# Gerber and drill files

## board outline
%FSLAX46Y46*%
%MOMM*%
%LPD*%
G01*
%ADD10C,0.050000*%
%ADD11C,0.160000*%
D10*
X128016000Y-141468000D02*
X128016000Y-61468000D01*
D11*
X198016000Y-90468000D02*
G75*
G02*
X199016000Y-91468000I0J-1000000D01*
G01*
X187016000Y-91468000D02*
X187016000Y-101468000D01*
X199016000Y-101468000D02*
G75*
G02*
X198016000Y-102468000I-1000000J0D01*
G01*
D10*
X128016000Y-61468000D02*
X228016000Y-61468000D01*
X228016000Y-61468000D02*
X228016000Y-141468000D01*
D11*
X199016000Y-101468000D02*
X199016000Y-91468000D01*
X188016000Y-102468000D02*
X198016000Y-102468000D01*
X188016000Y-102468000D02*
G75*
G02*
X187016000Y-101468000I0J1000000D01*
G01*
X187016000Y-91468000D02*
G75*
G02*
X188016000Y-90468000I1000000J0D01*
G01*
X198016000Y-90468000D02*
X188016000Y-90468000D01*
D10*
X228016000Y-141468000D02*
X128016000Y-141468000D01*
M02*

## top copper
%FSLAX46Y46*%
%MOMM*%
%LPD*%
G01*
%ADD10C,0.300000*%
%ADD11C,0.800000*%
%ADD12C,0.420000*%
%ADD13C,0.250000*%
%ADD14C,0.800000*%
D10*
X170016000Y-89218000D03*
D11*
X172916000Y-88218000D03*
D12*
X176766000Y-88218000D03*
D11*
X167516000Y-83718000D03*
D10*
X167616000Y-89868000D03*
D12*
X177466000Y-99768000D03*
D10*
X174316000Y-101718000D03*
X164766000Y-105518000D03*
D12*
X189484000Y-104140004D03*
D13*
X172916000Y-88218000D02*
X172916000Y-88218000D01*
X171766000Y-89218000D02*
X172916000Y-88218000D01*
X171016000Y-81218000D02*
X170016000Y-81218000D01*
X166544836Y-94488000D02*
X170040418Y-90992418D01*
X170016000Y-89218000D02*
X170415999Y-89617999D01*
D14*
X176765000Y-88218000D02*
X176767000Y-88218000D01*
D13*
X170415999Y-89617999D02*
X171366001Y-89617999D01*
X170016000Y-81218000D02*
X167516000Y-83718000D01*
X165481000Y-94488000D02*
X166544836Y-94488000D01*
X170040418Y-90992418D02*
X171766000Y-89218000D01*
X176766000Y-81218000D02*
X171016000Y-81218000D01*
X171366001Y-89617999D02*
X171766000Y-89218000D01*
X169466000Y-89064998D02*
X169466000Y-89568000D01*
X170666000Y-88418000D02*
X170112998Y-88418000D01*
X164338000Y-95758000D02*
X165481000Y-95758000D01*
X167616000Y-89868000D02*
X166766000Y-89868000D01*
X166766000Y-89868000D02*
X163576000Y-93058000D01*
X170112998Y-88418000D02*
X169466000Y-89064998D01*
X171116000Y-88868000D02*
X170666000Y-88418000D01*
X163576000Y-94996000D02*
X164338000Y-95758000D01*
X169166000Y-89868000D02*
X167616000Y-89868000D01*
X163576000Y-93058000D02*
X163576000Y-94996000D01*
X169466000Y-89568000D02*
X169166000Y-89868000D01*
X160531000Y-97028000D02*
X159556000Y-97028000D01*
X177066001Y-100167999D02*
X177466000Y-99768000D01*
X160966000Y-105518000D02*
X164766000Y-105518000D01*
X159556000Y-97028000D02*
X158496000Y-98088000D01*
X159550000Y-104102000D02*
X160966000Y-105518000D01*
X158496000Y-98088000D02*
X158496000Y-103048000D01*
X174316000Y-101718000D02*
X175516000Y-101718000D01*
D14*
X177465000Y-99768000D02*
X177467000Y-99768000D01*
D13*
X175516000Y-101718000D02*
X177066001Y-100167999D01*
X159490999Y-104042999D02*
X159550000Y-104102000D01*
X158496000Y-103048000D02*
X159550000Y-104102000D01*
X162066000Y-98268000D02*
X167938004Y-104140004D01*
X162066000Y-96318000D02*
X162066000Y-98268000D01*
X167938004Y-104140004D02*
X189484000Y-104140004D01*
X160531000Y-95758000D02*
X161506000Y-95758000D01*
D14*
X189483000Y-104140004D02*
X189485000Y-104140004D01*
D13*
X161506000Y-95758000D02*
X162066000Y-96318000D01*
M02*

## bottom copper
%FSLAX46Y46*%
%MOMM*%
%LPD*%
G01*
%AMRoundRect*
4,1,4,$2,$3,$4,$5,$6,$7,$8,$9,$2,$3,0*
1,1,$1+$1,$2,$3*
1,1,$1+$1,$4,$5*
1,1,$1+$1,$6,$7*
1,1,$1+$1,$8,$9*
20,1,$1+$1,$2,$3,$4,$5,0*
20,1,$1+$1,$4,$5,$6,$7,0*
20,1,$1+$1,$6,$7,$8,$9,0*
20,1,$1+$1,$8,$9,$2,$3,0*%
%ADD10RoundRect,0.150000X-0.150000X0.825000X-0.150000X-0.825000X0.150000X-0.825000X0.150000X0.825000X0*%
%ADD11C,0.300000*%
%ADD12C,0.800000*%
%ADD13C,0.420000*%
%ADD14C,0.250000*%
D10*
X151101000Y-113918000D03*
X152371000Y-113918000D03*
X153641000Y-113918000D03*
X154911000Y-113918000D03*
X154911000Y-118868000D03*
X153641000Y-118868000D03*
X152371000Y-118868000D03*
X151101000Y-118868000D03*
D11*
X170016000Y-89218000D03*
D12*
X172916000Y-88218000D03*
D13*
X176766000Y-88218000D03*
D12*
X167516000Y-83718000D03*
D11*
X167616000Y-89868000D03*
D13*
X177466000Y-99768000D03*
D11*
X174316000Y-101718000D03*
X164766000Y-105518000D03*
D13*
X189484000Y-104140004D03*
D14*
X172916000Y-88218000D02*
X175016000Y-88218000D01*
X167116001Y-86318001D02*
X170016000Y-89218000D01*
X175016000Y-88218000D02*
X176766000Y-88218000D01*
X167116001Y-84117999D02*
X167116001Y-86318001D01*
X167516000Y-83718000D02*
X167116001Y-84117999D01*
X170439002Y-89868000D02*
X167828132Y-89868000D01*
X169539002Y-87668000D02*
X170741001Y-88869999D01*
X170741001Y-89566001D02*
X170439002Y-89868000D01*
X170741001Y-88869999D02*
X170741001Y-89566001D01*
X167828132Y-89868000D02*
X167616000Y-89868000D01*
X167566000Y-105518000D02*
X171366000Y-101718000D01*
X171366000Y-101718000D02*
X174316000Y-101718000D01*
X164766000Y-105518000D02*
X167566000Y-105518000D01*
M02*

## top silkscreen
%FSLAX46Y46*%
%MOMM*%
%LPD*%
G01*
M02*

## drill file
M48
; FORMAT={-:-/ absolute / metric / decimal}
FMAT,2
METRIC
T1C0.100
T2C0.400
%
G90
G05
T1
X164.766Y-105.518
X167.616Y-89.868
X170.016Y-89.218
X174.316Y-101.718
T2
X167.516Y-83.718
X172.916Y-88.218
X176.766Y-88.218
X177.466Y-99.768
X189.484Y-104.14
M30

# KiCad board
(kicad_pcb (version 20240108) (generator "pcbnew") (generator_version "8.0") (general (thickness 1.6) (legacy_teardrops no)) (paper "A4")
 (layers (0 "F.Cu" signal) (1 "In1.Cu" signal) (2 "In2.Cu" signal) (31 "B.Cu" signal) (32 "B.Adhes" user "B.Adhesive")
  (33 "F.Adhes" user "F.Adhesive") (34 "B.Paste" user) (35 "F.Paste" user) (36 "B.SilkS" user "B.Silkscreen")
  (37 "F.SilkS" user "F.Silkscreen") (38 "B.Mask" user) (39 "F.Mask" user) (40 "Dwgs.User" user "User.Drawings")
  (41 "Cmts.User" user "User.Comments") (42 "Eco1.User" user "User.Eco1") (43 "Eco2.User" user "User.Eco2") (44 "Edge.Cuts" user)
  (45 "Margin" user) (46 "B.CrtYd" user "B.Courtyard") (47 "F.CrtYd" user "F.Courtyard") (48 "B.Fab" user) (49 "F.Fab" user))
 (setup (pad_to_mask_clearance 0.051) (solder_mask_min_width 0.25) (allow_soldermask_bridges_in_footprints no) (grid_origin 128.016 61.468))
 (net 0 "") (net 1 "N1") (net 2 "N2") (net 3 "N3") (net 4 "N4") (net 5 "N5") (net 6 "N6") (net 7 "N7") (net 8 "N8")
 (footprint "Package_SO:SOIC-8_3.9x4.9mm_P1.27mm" (layer "B.Cu") (at 153.006 116.393 -90)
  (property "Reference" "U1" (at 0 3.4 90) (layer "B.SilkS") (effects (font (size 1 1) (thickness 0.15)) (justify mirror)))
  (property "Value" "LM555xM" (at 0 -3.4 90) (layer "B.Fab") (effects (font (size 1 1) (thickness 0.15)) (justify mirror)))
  (pad "1" smd roundrect (at -2.475 1.905 270) (size 1.95 0.6) (layers "B.Cu" "B.Paste" "B.Mask") (roundrect_rratio 0.25) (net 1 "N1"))
  (pad "2" smd roundrect (at -2.475 0.635 270) (size 1.95 0.6) (layers "B.Cu" "B.Paste" "B.Mask") (roundrect_rratio 0.25) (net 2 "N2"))
  (pad "3" smd roundrect (at -2.475 -0.635 270) (size 1.95 0.6) (layers "B.Cu" "B.Paste" "B.Mask") (roundrect_rratio 0.25) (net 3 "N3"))
  (pad "4" smd roundrect (at -2.475 -1.905 270) (size 1.95 0.6) (layers "B.Cu" "B.Paste" "B.Mask") (roundrect_rratio 0.25) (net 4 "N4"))
  (pad "5" smd roundrect (at 2.475 -1.905 270) (size 1.95 0.6) (layers "B.Cu" "B.Paste" "B.Mask") (roundrect_rratio 0.25) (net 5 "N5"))
  (pad "6" smd roundrect (at 2.475 -0.635 270) (size 1.95 0.6) (layers "B.Cu" "B.Paste" "B.Mask") (roundrect_rratio 0.25) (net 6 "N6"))
  (pad "7" smd roundrect (at 2.475 0.635 270) (size 1.95 0.6) (layers "B.Cu" "B.Paste" "B.Mask") (roundrect_rratio 0.25) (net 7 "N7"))
  (pad "8" smd roundrect (at 2.475 1.905 270) (size 1.95 0.6) (layers "B.Cu" "B.Paste" "B.Mask") (roundrect_rratio 0.25) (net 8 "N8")))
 (gr_line (start 128.016 141.468) (end 128.016 61.468) (stroke (width 0.05) (type solid)) (layer "Edge.Cuts"))
 (gr_arc (start 198.016 90.468) (mid 198.723107 90.760893) (end 199.016 91.468) (stroke (width 0.16) (type solid)) (layer "Edge.Cuts"))
 (gr_line (start 187.016 91.468) (end 187.016 101.468) (stroke (width 0.16) (type solid)) (layer "Edge.Cuts"))
 (gr_arc (start 199.016 101.468) (mid 198.723107 102.175107) (end 198.016 102.468) (stroke (width 0.16) (type solid)) (layer "Edge.Cuts"))
 (gr_line (start 128.016 61.468) (end 228.016 61.468) (stroke (width 0.05) (type solid)) (layer "Edge.Cuts"))
 (gr_line (start 228.016 61.468) (end 228.016 141.468) (stroke (width 0.05) (type solid)) (layer "Edge.Cuts"))
 (gr_line (start 199.016 101.468) (end 199.016 91.468) (stroke (width 0.16) (type solid)) (layer "Edge.Cuts"))
 (gr_line (start 188.016 102.468) (end 198.016 102.468) (stroke (width 0.16) (type solid)) (layer "Edge.Cuts"))
 (gr_arc (start 188.016 102.468) (mid 187.308893 102.175107) (end 187.016 101.468) (stroke (width 0.16) (type solid)) (layer "Edge.Cuts"))
 (gr_arc (start 187.016 91.468) (mid 187.308893 90.760893) (end 188.016 90.468) (stroke (width 0.16) (type solid)) (layer "Edge.Cuts"))
 (gr_line (start 198.016 90.468) (end 188.016 90.468) (stroke (width 0.16) (type solid)) (layer "Edge.Cuts"))
 (gr_line (start 228.016 141.468) (end 128.016 141.468) (stroke (width 0.05) (type solid)) (layer "Edge.Cuts"))
 (segment (start 172.916 88.218) (end 172.916 88.218) (width 0.25) (layer "F.Cu") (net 8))
 (segment (start 171.766 89.218) (end 172.916 88.218) (width 0.25) (layer "F.Cu") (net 8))
 (segment (start 171.016 81.218) (end 170.016 81.218) (width 0.25) (layer "F.Cu") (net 8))
 (segment (start 166.544836 94.488) (end 170.040418 90.992418) (width 0.25) (layer "F.Cu") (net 8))
 (segment (start 170.016 89.218) (end 170.415999 89.617999) (width 0.25) (layer "F.Cu") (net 8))
 (segment (start 176.765 88.218) (end 176.767 88.218) (width 0.8) (layer "F.Cu") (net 8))
 (segment (start 170.415999 89.617999) (end 171.366001 89.617999) (width 0.25) (layer "F.Cu") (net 8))
 (segment (start 170.016 81.218) (end 167.516 83.718) (width 0.25) (layer "F.Cu") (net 8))
 (segment (start 165.481 94.488) (end 166.544836 94.488) (width 0.25) (layer "F.Cu") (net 8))
 (segment (start 170.040418 90.992418) (end 171.766 89.218) (width 0.25) (layer "F.Cu") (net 8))
 (segment (start 176.766 81.218) (end 171.016 81.218) (width 0.25) (layer "F.Cu") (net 8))
 (segment (start 171.366001 89.617999) (end 171.766 89.218) (width 0.25) (layer "F.Cu") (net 8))
 (via (at 170.016 89.218) (size 0.3) (drill 0.1) (layers "F.Cu" "B.Cu") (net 8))
 (via (at 172.916 88.218) (size 0.8) (drill 0.4) (layers "F.Cu" "B.Cu") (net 8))
 (via (at 176.766 88.218) (size 0.42) (drill 0.4) (layers "F.Cu" "B.Cu") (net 8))
 (via (at 167.516 83.718) (size 0.8) (drill 0.4) (layers "F.Cu" "B.Cu") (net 8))
 (segment (start 172.916 88.218) (end 175.016 88.218) (width 0.25) (layer "B.Cu") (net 8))
 (segment (start 167.116001 86.318001) (end 170.016 89.218) (width 0.25) (layer "B.Cu") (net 8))
 (segment (start 175.016 88.218) (end 176.766 88.218) (width 0.25) (layer "B.Cu") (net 8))
 (segment (start 167.116001 84.117999) (end 167.116001 86.318001) (width 0.25) (layer "B.Cu") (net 8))
 (segment (start 167.516 83.718) (end 167.116001 84.117999) (width 0.25) (layer "B.Cu") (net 8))
 (segment (start 169.466 89.064998) (end 169.466 89.568) (width 0.25) (layer "F.Cu") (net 7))
 (segment (start 170.666 88.418) (end 170.112998 88.418) (width 0.25) (layer "F.Cu") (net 7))
 (segment (start 164.338 95.758) (end 165.481 95.758) (width 0.25) (layer "F.Cu") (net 7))
 (segment (start 167.616 89.868) (end 166.766 89.868) (width 0.25) (layer "F.Cu") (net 7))
 (segment (start 166.766 89.868) (end 163.576 93.058) (width 0.25) (layer "F.Cu") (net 7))
 (segment (start 170.112998 88.418) (end 169.466 89.064998) (width 0.25) (layer "F.Cu") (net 7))
 (segment (start 171.116 88.868) (end 170.666 88.418) (width 0.25) (layer "F.Cu") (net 7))
 (segment (start 163.576 94.996) (end 164.338 95.758) (width 0.25) (layer "F.Cu") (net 7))
 (segment (start 169.166 89.868) (end 167.616 89.868) (width 0.25) (layer "F.Cu") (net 7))
 (segment (start 163.576 93.058) (end 163.576 94.996) (width 0.25) (layer "F.Cu") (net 7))
 (segment (start 169.466 89.568) (end 169.166 89.868) (width 0.25) (layer "F.Cu") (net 7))
 (via (at 167.616 89.868) (size 0.3) (drill 0.1) (layers "F.Cu" "B.Cu") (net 7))
 (segment (start 170.439002 89.868) (end 167.828132 89.868) (width 0.25) (layer "B.Cu") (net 7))
 (segment (start 169.539002 87.668) (end 170.741001 88.869999) (width 0.25) (layer "B.Cu") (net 7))
 (segment (start 170.741001 89.566001) (end 170.439002 89.868) (width 0.25) (layer "B.Cu") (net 7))
 (segment (start 170.741001 88.869999) (end 170.741001 89.566001) (width 0.25) (layer "B.Cu") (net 7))
 (segment (start 167.828132 89.868) (end 167.616 89.868) (width 0.25) (layer "B.Cu") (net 7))
 (segment (start 160.531 97.028) (end 159.556 97.028) (width 0.25) (layer "F.Cu") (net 3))
 (segment (start 177.066001 100.167999) (end 177.466 99.768) (width 0.25) (layer "F.Cu") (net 3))
 (segment (start 160.966 105.518) (end 164.766 105.518) (width 0.25) (layer "F.Cu") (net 3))
 (segment (start 159.556 97.028) (end 158.496 98.088) (width 0.25) (layer "F.Cu") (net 3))
 (segment (start 159.55 104.102) (end 160.966 105.518) (width 0.25) (layer "F.Cu") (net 3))
 (segment (start 158.496 98.088) (end 158.496 103.048) (width 0.25) (layer "F.Cu") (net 3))
 (segment (start 174.316 101.718) (end 175.516 101.718) (width 0.25) (layer "F.Cu") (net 3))
 (segment (start 177.465 99.768) (end 177.467 99.768) (width 0.8) (layer "F.Cu") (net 3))
 (segment (start 175.516 101.718) (end 177.066001 100.167999) (width 0.25) (layer "F.Cu") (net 3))
 (segment (start 159.490999 104.042999) (end 159.55 104.102) (width 0.25) (layer "F.Cu") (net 3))
 (segment (start 158.496 103.048) (end 159.55 104.102) (width 0.25) (layer "F.Cu") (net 3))
 (via (at 177.466 99.768) (size 0.42) (drill 0.4) (layers "F.Cu" "B.Cu") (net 3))
 (via (at 174.316 101.718) (size 0.3) (drill 0.1) (layers "F.Cu" "B.Cu") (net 3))
 (via (at 164.766 105.518) (size 0.3) (drill 0.1) (layers "F.Cu" "B.Cu") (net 3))
 (segment (start 167.566 105.518) (end 171.366 101.718) (width 0.25) (layer "B.Cu") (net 3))
 (segment (start 171.366 101.718) (end 174.316 101.718) (width 0.25) (layer "B.Cu") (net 3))
 (segment (start 164.766 105.518) (end 167.566 105.518) (width 0.25) (layer "B.Cu") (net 3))
 (segment (start 162.066 98.268) (end 167.938004 104.140004) (width 0.25) (layer "F.Cu") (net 2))
 (segment (start 162.066 96.318) (end 162.066 98.268) (width 0.25) (layer "F.Cu") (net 2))
 (segment (start 167.938004 104.140004) (end 189.484 104.140004) (width 0.25) (layer "F.Cu") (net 2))
 (segment (start 160.531 95.758) (end 161.506 95.758) (width 0.25) (layer "F.Cu") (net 2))
 (segment (start 189.483 104.140004) (end 189.485 104.140004) (width 0.8) (layer "F.Cu") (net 2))
 (segment (start 161.506 95.758) (end 162.066 96.318) (width 0.25) (layer "F.Cu") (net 2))
 (via (at 189.484 104.140004) (size 0.42) (drill 0.4) (layers "F.Cu" "B.Cu") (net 2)))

